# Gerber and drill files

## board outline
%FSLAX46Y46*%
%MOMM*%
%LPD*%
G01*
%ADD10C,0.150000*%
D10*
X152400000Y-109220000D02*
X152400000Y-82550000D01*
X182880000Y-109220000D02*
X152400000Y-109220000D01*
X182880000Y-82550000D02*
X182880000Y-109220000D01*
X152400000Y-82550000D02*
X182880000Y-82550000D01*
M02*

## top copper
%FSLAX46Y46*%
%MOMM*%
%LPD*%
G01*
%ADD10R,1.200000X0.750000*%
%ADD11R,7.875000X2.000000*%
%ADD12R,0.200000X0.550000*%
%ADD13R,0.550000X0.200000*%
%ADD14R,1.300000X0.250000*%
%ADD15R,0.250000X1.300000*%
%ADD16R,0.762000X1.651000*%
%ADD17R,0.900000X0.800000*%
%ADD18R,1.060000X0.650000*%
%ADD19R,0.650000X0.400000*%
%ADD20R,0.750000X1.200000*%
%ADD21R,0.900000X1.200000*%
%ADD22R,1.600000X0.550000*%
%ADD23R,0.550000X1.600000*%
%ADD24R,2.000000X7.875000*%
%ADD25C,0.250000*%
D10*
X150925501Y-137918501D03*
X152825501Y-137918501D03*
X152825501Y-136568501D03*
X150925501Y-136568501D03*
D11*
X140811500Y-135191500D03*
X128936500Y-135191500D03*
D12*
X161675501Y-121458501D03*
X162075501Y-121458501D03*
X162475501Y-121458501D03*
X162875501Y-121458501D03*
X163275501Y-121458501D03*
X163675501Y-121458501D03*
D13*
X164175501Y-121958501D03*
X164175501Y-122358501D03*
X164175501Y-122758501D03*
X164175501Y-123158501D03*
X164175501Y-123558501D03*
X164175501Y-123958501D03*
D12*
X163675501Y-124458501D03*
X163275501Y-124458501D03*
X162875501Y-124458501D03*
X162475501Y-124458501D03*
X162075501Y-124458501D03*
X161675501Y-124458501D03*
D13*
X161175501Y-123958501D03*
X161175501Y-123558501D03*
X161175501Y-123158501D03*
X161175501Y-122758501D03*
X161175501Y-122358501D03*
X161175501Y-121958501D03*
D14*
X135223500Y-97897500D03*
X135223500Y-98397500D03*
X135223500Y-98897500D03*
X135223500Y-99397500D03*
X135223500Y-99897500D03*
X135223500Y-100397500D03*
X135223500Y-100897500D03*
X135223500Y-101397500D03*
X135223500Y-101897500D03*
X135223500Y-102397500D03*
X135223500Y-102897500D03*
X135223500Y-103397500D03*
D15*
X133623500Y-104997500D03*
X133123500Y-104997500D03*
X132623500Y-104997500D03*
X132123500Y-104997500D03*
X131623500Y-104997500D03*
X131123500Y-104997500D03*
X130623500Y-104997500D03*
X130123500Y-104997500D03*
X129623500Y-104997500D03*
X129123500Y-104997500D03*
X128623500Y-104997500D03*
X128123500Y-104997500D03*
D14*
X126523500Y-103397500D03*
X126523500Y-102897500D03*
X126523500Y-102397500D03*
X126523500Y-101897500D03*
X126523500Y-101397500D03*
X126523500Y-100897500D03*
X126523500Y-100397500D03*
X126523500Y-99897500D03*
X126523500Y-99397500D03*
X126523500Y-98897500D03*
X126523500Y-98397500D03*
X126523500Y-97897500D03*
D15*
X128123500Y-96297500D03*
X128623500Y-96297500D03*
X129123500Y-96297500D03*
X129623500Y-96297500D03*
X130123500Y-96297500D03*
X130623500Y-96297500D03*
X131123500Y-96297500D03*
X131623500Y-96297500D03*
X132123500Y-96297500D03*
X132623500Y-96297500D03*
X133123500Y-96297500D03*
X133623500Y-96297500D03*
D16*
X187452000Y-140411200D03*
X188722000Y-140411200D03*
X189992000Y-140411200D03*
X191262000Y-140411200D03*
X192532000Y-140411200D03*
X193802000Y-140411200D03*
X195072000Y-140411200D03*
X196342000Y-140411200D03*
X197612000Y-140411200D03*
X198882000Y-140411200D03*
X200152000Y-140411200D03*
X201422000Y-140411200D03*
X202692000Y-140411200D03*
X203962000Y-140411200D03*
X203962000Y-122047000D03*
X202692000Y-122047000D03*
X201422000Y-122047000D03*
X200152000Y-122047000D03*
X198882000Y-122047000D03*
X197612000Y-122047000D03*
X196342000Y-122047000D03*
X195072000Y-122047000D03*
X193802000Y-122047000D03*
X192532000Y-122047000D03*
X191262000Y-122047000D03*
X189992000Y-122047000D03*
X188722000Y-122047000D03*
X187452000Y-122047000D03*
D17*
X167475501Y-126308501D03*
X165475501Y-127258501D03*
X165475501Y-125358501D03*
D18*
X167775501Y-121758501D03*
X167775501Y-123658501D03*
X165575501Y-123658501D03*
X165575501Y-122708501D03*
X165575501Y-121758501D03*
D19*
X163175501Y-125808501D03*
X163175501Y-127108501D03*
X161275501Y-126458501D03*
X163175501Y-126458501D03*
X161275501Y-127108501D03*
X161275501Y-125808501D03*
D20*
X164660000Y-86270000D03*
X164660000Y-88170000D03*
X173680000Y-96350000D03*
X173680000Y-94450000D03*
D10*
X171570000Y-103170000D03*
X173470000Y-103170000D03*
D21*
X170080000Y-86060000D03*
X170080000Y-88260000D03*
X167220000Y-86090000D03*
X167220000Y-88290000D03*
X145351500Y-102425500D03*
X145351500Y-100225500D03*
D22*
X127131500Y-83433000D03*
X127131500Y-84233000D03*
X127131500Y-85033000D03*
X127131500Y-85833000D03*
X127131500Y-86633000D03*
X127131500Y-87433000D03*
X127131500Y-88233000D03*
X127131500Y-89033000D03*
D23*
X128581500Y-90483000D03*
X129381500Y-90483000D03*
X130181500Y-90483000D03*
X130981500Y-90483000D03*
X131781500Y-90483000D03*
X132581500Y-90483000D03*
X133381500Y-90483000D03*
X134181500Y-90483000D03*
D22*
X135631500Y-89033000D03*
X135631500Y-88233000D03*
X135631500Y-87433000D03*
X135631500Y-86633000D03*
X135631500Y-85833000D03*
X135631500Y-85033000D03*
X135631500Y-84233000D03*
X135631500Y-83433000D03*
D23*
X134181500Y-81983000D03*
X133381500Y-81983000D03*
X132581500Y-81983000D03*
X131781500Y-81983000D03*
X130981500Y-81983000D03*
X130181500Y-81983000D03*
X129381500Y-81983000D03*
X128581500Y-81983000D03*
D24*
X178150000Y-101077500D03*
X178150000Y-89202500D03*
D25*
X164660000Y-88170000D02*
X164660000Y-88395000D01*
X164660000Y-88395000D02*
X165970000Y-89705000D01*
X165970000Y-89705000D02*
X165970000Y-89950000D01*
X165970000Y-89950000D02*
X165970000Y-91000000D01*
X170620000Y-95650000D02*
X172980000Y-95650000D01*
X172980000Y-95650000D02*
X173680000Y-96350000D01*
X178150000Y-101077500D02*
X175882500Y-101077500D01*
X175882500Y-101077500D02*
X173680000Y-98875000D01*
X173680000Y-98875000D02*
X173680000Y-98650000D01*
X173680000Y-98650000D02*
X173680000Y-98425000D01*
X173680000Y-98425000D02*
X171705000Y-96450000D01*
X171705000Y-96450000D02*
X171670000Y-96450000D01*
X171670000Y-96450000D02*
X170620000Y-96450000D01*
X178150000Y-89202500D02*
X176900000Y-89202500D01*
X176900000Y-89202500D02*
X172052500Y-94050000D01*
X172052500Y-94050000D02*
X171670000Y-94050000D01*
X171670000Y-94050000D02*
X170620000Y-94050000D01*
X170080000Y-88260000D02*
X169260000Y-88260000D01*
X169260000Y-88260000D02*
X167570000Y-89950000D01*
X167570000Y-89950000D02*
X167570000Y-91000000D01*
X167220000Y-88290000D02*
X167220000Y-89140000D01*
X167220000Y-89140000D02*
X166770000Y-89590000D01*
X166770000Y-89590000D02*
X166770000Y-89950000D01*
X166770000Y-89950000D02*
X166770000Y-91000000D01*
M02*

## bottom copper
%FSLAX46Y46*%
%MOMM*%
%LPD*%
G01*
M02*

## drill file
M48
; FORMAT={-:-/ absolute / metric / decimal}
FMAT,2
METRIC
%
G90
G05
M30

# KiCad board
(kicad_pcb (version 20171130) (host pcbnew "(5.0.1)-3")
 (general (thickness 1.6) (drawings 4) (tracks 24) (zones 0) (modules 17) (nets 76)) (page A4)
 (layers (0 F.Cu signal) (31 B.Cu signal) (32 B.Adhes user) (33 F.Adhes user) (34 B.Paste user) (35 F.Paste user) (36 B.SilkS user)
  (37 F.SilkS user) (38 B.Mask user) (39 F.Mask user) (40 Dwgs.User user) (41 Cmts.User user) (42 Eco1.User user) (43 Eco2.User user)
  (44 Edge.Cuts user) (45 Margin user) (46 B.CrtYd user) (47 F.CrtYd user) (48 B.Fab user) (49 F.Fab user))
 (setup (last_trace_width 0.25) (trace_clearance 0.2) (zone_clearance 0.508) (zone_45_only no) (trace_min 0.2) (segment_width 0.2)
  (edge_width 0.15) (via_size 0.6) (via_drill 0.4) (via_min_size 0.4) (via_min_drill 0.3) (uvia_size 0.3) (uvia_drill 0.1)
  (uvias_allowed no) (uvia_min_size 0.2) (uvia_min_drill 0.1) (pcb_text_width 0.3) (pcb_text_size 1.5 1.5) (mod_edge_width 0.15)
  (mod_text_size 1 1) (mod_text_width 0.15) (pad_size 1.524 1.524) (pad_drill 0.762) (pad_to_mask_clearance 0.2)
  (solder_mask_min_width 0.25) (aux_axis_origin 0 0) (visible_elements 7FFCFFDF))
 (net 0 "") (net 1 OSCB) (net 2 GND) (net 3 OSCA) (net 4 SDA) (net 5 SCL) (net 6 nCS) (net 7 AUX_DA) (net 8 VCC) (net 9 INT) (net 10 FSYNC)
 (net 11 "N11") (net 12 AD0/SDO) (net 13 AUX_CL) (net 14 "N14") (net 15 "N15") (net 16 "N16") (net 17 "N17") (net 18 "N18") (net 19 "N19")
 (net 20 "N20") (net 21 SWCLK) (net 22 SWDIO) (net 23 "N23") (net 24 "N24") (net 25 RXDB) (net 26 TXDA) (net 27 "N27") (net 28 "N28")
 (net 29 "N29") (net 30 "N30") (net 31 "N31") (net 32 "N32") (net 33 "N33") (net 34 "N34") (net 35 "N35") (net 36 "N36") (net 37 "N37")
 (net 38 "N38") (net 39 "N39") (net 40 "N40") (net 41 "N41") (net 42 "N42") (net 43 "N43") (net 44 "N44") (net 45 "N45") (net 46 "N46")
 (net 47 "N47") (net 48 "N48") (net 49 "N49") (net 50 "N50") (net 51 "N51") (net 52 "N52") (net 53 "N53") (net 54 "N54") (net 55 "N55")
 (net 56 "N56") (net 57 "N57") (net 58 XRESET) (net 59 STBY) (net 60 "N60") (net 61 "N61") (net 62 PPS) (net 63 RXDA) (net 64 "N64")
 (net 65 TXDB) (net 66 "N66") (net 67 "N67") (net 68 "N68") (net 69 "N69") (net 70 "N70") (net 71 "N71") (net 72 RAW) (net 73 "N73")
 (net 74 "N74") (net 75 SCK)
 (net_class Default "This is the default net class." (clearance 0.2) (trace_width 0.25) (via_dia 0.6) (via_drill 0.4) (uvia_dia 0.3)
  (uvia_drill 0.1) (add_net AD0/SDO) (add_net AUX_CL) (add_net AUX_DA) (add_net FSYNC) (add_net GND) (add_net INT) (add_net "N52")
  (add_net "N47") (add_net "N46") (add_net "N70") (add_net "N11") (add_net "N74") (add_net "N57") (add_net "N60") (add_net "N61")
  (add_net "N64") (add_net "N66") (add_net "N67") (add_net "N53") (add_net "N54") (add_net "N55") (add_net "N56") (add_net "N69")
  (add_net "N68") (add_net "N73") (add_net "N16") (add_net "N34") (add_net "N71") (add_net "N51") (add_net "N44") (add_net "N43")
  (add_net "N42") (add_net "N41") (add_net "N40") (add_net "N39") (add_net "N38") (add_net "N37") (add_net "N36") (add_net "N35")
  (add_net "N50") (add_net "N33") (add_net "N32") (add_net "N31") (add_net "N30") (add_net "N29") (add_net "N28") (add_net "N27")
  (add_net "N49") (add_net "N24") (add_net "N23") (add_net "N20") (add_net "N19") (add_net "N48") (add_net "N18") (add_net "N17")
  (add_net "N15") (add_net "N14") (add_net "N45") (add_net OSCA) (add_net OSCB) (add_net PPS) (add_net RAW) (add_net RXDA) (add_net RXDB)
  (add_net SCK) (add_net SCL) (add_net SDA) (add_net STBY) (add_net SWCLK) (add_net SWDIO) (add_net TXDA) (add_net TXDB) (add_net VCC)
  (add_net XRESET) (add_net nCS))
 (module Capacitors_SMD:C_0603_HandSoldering (layer F.Cu) (at 151.875501 137.918501)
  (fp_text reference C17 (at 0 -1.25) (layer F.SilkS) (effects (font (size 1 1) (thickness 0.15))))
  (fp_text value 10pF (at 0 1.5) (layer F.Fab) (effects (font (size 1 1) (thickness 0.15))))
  (pad 1 smd rect (at -0.95 0) (size 1.2 0.75) (layers F.Cu F.Paste F.Mask) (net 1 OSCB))
  (pad 2 smd rect (at 0.95 0) (size 1.2 0.75) (layers F.Cu F.Paste F.Mask) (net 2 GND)))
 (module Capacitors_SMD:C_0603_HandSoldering (layer F.Cu) (at 151.875501 136.568501)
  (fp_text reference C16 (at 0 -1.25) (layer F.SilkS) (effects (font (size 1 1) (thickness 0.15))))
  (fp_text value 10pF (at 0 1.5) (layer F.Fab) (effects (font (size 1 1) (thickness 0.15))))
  (pad 2 smd rect (at 0.95 0) (size 1.2 0.75) (layers F.Cu F.Paste F.Mask) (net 2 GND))
  (pad 1 smd rect (at -0.95 0) (size 1.2 0.75) (layers F.Cu F.Paste F.Mask) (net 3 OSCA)))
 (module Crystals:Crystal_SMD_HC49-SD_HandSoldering (layer F.Cu) (at 134.874 135.1915)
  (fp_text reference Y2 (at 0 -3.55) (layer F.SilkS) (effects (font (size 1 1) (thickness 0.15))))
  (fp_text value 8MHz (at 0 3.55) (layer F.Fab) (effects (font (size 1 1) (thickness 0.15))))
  (pad 2 smd rect (at 5.9375 0) (size 7.875 2) (layers F.Cu F.Paste F.Mask) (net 1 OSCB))
  (pad 1 smd rect (at -5.9375 0) (size 7.875 2) (layers F.Cu F.Paste F.Mask) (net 3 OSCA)))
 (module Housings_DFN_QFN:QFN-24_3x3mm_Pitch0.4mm (layer F.Cu) (at 162.675501 122.958501)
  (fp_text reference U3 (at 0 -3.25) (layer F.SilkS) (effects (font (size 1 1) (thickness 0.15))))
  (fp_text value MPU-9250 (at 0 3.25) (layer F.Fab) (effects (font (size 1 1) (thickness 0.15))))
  (pad 24 smd rect (at -1 -1.5 90) (size 0.55 0.2) (layers F.Cu F.Paste F.Mask) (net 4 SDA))
  (pad 23 smd rect (at -0.6 -1.5 90) (size 0.55 0.2) (layers F.Cu F.Paste F.Mask) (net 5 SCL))
  (pad 22 smd rect (at -0.2 -1.5 90) (size 0.55 0.2) (layers F.Cu F.Paste F.Mask) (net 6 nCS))
  (pad 21 smd rect (at 0.2 -1.5 90) (size 0.55 0.2) (layers F.Cu F.Paste F.Mask) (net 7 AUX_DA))
  (pad 20 smd rect (at 0.6 -1.5 90) (size 0.55 0.2) (layers F.Cu F.Paste F.Mask))
  (pad 19 smd rect (at 1 -1.5 90) (size 0.55 0.2) (layers F.Cu F.Paste F.Mask))
  (pad 18 smd rect (at 1.5 -1) (size 0.55 0.2) (layers F.Cu F.Paste F.Mask) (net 2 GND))
  (pad 17 smd rect (at 1.5 -0.6) (size 0.55 0.2) (layers F.Cu F.Paste F.Mask))
  (pad 16 smd rect (at 1.5 -0.2) (size 0.55 0.2) (layers F.Cu F.Paste F.Mask))
  (pad 15 smd rect (at 1.5 0.2) (size 0.55 0.2) (layers F.Cu F.Paste F.Mask))
  (pad 14 smd rect (at 1.5 0.6) (size 0.55 0.2) (layers F.Cu F.Paste F.Mask))
  (pad 13 smd rect (at 1.5 1) (size 0.55 0.2) (layers F.Cu F.Paste F.Mask) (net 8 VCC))
  (pad 12 smd rect (at 1 1.5 90) (size 0.55 0.2) (layers F.Cu F.Paste F.Mask) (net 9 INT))
  (pad 11 smd rect (at 0.6 1.5 90) (size 0.55 0.2) (layers F.Cu F.Paste F.Mask) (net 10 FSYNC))
  (pad 10 smd rect (at 0.2 1.5 90) (size 0.55 0.2) (layers F.Cu F.Paste F.Mask) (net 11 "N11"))
  (pad 9 smd rect (at -0.2 1.5 90) (size 0.55 0.2) (layers F.Cu F.Paste F.Mask) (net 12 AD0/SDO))
  (pad 8 smd rect (at -0.6 1.5 90) (size 0.55 0.2) (layers F.Cu F.Paste F.Mask) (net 8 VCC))
  (pad 7 smd rect (at -1 1.5 90) (size 0.55 0.2) (layers F.Cu F.Paste F.Mask) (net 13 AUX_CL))
  (pad 6 smd rect (at -1.5 1) (size 0.55 0.2) (layers F.Cu F.Paste F.Mask))
  (pad 5 smd rect (at -1.5 0.6) (size 0.55 0.2) (layers F.Cu F.Paste F.Mask))
  (pad 4 smd rect (at -1.5 0.2) (size 0.55 0.2) (layers F.Cu F.Paste F.Mask))
  (pad 3 smd rect (at -1.5 -0.2) (size 0.55 0.2) (layers F.Cu F.Paste F.Mask))
  (pad 2 smd rect (at -1.5 -0.6) (size 0.55 0.2) (layers F.Cu F.Paste F.Mask))
  (pad 1 smd rect (at -1.5 -1) (size 0.55 0.2) (layers F.Cu F.Paste F.Mask)))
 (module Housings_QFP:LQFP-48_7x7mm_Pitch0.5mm (layer F.Cu) (at 130.8735 100.6475 270)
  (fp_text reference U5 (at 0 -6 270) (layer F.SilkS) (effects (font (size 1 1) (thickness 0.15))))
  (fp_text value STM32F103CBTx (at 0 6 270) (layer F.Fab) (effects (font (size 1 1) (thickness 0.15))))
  (pad 48 smd rect (at -2.75 -4.35) (size 1.3 0.25) (layers F.Cu F.Paste F.Mask) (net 8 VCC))
  (pad 47 smd rect (at -2.25 -4.35) (size 1.3 0.25) (layers F.Cu F.Paste F.Mask) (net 2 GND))
  (pad 46 smd rect (at -1.75 -4.35) (size 1.3 0.25) (layers F.Cu F.Paste F.Mask) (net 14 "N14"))
  (pad 45 smd rect (at -1.25 -4.35) (size 1.3 0.25) (layers F.Cu F.Paste F.Mask) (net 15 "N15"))
  (pad 44 smd rect (at -0.75 -4.35) (size 1.3 0.25) (layers F.Cu F.Paste F.Mask) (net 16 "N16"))
  (pad 43 smd rect (at -0.25 -4.35) (size 1.3 0.25) (layers F.Cu F.Paste F.Mask) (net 4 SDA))
  (pad 42 smd rect (at 0.25 -4.35) (size 1.3 0.25) (layers F.Cu F.Paste F.Mask) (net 5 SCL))
  (pad 41 smd rect (at 0.75 -4.35) (size 1.3 0.25) (layers F.Cu F.Paste F.Mask) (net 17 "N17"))
  (pad 40 smd rect (at 1.25 -4.35) (size 1.3 0.25) (layers F.Cu F.Paste F.Mask) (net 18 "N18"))
  (pad 39 smd rect (at 1.75 -4.35) (size 1.3 0.25) (layers F.Cu F.Paste F.Mask) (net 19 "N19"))
  (pad 38 smd rect (at 2.25 -4.35) (size 1.3 0.25) (layers F.Cu F.Paste F.Mask) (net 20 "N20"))
  (pad 37 smd rect (at 2.75 -4.35) (size 1.3 0.25) (layers F.Cu F.Paste F.Mask) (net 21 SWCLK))
  (pad 36 smd rect (at 4.35 -2.75 270) (size 1.3 0.25) (layers F.Cu F.Paste F.Mask) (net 8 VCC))
  (pad 35 smd rect (at 4.35 -2.25 270) (size 1.3 0.25) (layers F.Cu F.Paste F.Mask) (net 2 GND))
  (pad 34 smd rect (at 4.35 -1.75 270) (size 1.3 0.25) (layers F.Cu F.Paste F.Mask) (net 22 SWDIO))
  (pad 33 smd rect (at 4.35 -1.25 270) (size 1.3 0.25) (layers F.Cu F.Paste F.Mask) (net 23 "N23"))
  (pad 32 smd rect (at 4.35 -0.75 270) (size 1.3 0.25) (layers F.Cu F.Paste F.Mask) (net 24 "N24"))
  (pad 31 smd rect (at 4.35 -0.25 270) (size 1.3 0.25) (layers F.Cu F.Paste F.Mask) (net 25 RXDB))
  (pad 30 smd rect (at 4.35 0.25 270) (size 1.3 0.25) (layers F.Cu F.Paste F.Mask) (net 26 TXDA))
  (pad 29 smd rect (at 4.35 0.75 270) (size 1.3 0.25) (layers F.Cu F.Paste F.Mask) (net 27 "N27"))
  (pad 28 smd rect (at 4.35 1.25 270) (size 1.3 0.25) (layers F.Cu F.Paste F.Mask) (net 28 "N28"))
  (pad 27 smd rect (at 4.35 1.75 270) (size 1.3 0.25) (layers F.Cu F.Paste F.Mask) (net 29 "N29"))
  (pad 26 smd rect (at 4.35 2.25 270) (size 1.3 0.25) (layers F.Cu F.Paste F.Mask) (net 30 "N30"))
  (pad 25 smd rect (at 4.35 2.75 270) (size 1.3 0.25) (layers F.Cu F.Paste F.Mask) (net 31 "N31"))
  (pad 24 smd rect (at 2.75 4.35) (size 1.3 0.25) (layers F.Cu F.Paste F.Mask) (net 8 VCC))
  (pad 23 smd rect (at 2.25 4.35) (size 1.3 0.25) (layers F.Cu F.Paste F.Mask) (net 2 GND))
  (pad 22 smd rect (at 1.75 4.35) (size 1.3 0.25) (layers F.Cu F.Paste F.Mask) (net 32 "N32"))
  (pad 21 smd rect (at 1.25 4.35) (size 1.3 0.25) (layers F.Cu F.Paste F.Mask) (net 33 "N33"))
  (pad 20 smd rect (at 0.75 4.35) (size 1.3 0.25) (layers F.Cu F.Paste F.Mask) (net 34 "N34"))
  (pad 19 smd rect (at 0.25 4.35) (size 1.3 0.25) (layers F.Cu F.Paste F.Mask) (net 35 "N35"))
  (pad 18 smd rect (at -0.25 4.35) (size 1.3 0.25) (layers F.Cu F.Paste F.Mask) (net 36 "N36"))
  (pad 17 smd rect (at -0.75 4.35) (size 1.3 0.25) (layers F.Cu F.Paste F.Mask) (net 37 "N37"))
  (pad 16 smd rect (at -1.25 4.35) (size 1.3 0.25) (layers F.Cu F.Paste F.Mask) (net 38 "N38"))
  (pad 15 smd rect (at -1.75 4.35) (size 1.3 0.25) (layers F.Cu F.Paste F.Mask) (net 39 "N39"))
  (pad 14 smd rect (at -2.25 4.35) (size 1.3 0.25) (layers F.Cu F.Paste F.Mask) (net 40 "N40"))
  (pad 13 smd rect (at -2.75 4.35) (size 1.3 0.25) (layers F.Cu F.Paste F.Mask) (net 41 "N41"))
  (pad 12 smd rect (at -4.35 2.75 270) (size 1.3 0.25) (layers F.Cu F.Paste F.Mask) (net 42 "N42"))
  (pad 11 smd rect (at -4.35 2.25 270) (size 1.3 0.25) (layers F.Cu F.Paste F.Mask) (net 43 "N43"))
  (pad 10 smd rect (at -4.35 1.75 270) (size 1.3 0.25) (layers F.Cu F.Paste F.Mask) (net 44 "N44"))
  (pad 9 smd rect (at -4.35 1.25 270) (size 1.3 0.25) (layers F.Cu F.Paste F.Mask) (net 8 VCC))
  (pad 8 smd rect (at -4.35 0.75 270) (size 1.3 0.25) (layers F.Cu F.Paste F.Mask) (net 2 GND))
  (pad 7 smd rect (at -4.35 0.25 270) (size 1.3 0.25) (layers F.Cu F.Paste F.Mask) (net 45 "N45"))
  (pad 6 smd rect (at -4.35 -0.25 270) (size 1.3 0.25) (layers F.Cu F.Paste F.Mask) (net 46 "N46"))
  (pad 5 smd rect (at -4.35 -0.75 270) (size 1.3 0.25) (layers F.Cu F.Paste F.Mask) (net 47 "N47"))
  (pad 4 smd rect (at -4.35 -1.25 270) (size 1.3 0.25) (layers F.Cu F.Paste F.Mask) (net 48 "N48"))
  (pad 3 smd rect (at -4.35 -1.75 270) (size 1.3 0.25) (layers F.Cu F.Paste F.Mask) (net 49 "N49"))
  (pad 2 smd rect (at -4.35 -2.25 270) (size 1.3 0.25) (layers F.Cu F.Paste F.Mask) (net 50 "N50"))
  (pad 1 smd rect (at -4.35 -2.75 270) (size 1.3 0.25) (layers F.Cu F.Paste F.Mask) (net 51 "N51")))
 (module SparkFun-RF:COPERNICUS (layer F.Cu) (at 187.452 122.047)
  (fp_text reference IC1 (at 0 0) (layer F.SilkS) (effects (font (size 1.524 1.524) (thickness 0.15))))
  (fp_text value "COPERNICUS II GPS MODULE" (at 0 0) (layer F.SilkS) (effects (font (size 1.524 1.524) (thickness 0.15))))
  (pad 1 smd rect (at 0 18.3642 180) (size 0.762 1.651) (layers F.Cu F.Paste F.Mask) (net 2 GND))
  (pad 2 smd rect (at 1.27 18.3642 180) (size 0.762 1.651) (layers F.Cu F.Paste F.Mask) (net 2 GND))
  (pad 3 smd rect (at 2.54 18.3642 180) (size 0.762 1.651) (layers F.Cu F.Paste F.Mask) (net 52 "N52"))
  (pad 4 smd rect (at 3.81 18.3642 180) (size 0.762 1.651) (layers F.Cu F.Paste F.Mask) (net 2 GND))
  (pad 5 smd rect (at 5.08 18.3642 180) (size 0.762 1.651) (layers F.Cu F.Paste F.Mask) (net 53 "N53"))
  (pad 6 smd rect (at 6.35 18.3642 180) (size 0.762 1.651) (layers F.Cu F.Paste F.Mask) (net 8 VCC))
  (pad 7 smd rect (at 7.62 18.3642 180) (size 0.762 1.651) (layers F.Cu F.Paste F.Mask) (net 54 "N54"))
  (pad 8 smd rect (at 8.89 18.3642 180) (size 0.762 1.651) (layers F.Cu F.Paste F.Mask) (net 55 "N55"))
  (pad 9 smd rect (at 10.16 18.3642 180) (size 0.762 1.651) (layers F.Cu F.Paste F.Mask) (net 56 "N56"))
  (pad 10 smd rect (at 11.43 18.3642 180) (size 0.762 1.651) (layers F.Cu F.Paste F.Mask) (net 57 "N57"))
  (pad 11 smd rect (at 12.7 18.3642 180) (size 0.762 1.651) (layers F.Cu F.Paste F.Mask) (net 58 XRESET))
  (pad 12 smd rect (at 13.97 18.3642 180) (size 0.762 1.651) (layers F.Cu F.Paste F.Mask) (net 8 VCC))
  (pad 13 smd rect (at 15.24 18.3642 180) (size 0.762 1.651) (layers F.Cu F.Paste F.Mask) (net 2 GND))
  (pad 14 smd rect (at 16.51 18.3642 180) (size 0.762 1.651) (layers F.Cu F.Paste F.Mask) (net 2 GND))
  (pad 15 smd rect (at 16.51 0 180) (size 0.762 1.651) (layers F.Cu F.Paste F.Mask) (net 2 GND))
  (pad 16 smd rect (at 15.24 0 180) (size 0.762 1.651) (layers F.Cu F.Paste F.Mask) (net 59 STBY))
  (pad 17 smd rect (at 13.97 0 180) (size 0.762 1.651) (layers F.Cu F.Paste F.Mask) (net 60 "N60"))
  (pad 18 smd rect (at 12.7 0 180) (size 0.762 1.651) (layers F.Cu F.Paste F.Mask) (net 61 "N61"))
  (pad 19 smd rect (at 11.43 0 180) (size 0.762 1.651) (layers F.Cu F.Paste F.Mask) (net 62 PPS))
  (pad 20 smd rect (at 10.16 0 180) (size 0.762 1.651) (layers F.Cu F.Paste F.Mask) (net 25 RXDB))
  (pad 21 smd rect (at 8.89 0 180) (size 0.762 1.651) (layers F.Cu F.Paste F.Mask) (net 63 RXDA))
  (pad 22 smd rect (at 7.62 0 180) (size 0.762 1.651) (layers F.Cu F.Paste F.Mask) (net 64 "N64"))
  (pad 23 smd rect (at 6.35 0 180) (size 0.762 1.651) (layers F.Cu F.Paste F.Mask) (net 26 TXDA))
  (pad 24 smd rect (at 5.08 0 180) (size 0.762 1.651) (layers F.Cu F.Paste F.Mask) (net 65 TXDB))
  (pad 25 smd rect (at 3.81 0 180) (size 0.762 1.651) (layers F.Cu F.Paste F.Mask) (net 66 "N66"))
  (pad 26 smd rect (at 2.54 0 180) (size 0.762 1.651) (layers F.Cu F.Paste F.Mask) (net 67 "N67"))
  (pad 27 smd rect (at 1.27 0 180) (size 0.762 1.651) (layers F.Cu F.Paste F.Mask) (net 2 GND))
  (pad 28 smd rect (at 0 0 180) (size 0.762 1.651) (layers F.Cu F.Paste F.Mask) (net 2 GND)))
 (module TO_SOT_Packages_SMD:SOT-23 (layer F.Cu) (at 166.475501 126.308501)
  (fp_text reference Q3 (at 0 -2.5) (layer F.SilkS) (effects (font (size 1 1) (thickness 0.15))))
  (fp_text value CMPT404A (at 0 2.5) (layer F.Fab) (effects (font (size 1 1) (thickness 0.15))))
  (pad 3 smd rect (at 1 0) (size 0.9 0.8) (layers F.Cu F.Paste F.Mask) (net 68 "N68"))
  (pad 2 smd rect (at -1 0.95) (size 0.9 0.8) (layers F.Cu F.Paste F.Mask) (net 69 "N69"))
  (pad 1 smd rect (at -1 -0.95) (size 0.9 0.8) (layers F.Cu F.Paste F.Mask) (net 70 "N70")))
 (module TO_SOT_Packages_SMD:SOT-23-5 (layer F.Cu) (at 166.675501 122.708501)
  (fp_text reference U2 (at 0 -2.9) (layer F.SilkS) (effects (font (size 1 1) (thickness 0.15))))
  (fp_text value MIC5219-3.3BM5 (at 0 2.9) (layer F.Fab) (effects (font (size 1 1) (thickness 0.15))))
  (pad 5 smd rect (at 1.1 -0.95) (size 1.06 0.65) (layers F.Cu F.Paste F.Mask) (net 8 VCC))
  (pad 4 smd rect (at 1.1 0.95) (size 1.06 0.65) (layers F.Cu F.Paste F.Mask) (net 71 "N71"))
  (pad 3 smd rect (at -1.1 0.95) (size 1.06 0.65) (layers F.Cu F.Paste F.Mask) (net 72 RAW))
  (pad 2 smd rect (at -1.1 0) (size 1.06 0.65) (layers F.Cu F.Paste F.Mask) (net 2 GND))
  (pad 1 smd rect (at -1.1 -0.95) (size 1.06 0.65) (layers F.Cu F.Paste F.Mask) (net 72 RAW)))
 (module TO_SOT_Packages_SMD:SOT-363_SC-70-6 (layer F.Cu) (at 162.225501 126.458501)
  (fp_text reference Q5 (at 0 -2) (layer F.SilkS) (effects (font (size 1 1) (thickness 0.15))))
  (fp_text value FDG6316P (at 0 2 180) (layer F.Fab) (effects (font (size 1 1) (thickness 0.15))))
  (pad 6 smd rect (at 0.95 -0.65) (size 0.65 0.4) (layers F.Cu F.Paste F.Mask))
  (pad 4 smd rect (at 0.95 0.65) (size 0.65 0.4) (layers F.Cu F.Paste F.Mask))
  (pad 2 smd rect (at -0.95 0) (size 0.65 0.4) (layers F.Cu F.Paste F.Mask) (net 53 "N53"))
  (pad 5 smd rect (at 0.95 0) (size 0.65 0.4) (layers F.Cu F.Paste F.Mask))
  (pad 3 smd rect (at -0.95 0.65) (size 0.65 0.4) (layers F.Cu F.Paste F.Mask) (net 8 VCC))
  (pad 1 smd rect (at -0.95 -0.65) (size 0.65 0.4) (layers F.Cu F.Paste F.Mask) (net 69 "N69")))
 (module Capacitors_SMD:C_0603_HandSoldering (layer F.Cu) (at 164.66 87.22 270)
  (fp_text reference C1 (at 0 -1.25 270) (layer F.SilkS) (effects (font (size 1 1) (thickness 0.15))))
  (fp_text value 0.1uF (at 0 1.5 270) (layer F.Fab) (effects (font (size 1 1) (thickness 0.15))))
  (pad 1 smd rect (at -0.95 0 270) (size 1.2 0.75) (layers F.Cu F.Paste F.Mask) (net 8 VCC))
  (pad 2 smd rect (at 0.95 0 270) (size 1.2 0.75) (layers F.Cu F.Paste F.Mask) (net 2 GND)))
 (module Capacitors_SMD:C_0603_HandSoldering (layer F.Cu) (at 173.68 95.4 90)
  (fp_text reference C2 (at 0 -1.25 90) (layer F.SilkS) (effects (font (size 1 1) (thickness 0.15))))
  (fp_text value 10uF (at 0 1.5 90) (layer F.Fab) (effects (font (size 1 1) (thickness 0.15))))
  (pad 1 smd rect (at -0.95 0 90) (size 1.2 0.75) (layers F.Cu F.Paste F.Mask) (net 72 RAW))
  (pad 2 smd rect (at 0.95 0 90) (size 1.2 0.75) (layers F.Cu F.Paste F.Mask) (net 2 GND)))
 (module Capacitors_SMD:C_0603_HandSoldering (layer F.Cu) (at 172.52 103.17)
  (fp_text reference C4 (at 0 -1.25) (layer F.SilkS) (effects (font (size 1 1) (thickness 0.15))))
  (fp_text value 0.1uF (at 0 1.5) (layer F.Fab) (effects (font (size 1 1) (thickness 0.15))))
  (pad 1 smd rect (at -0.95 0) (size 1.2 0.75) (layers F.Cu F.Paste F.Mask) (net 11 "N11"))
  (pad 2 smd rect (at 0.95 0) (size 1.2 0.75) (layers F.Cu F.Paste F.Mask) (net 2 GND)))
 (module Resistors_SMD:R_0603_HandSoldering (layer F.Cu) (at 170.08 87.16 270)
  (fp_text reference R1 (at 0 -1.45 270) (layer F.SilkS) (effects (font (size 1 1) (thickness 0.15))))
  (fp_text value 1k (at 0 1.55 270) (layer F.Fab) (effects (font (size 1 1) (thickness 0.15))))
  (pad 1 smd rect (at -1.1 0 270) (size 1.2 0.9) (layers F.Cu F.Paste F.Mask) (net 70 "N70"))
  (pad 2 smd rect (at 1.1 0 270) (size 1.2 0.9) (layers F.Cu F.Paste F.Mask) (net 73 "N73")))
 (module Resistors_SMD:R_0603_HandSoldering (layer F.Cu) (at 167.22 87.19 270)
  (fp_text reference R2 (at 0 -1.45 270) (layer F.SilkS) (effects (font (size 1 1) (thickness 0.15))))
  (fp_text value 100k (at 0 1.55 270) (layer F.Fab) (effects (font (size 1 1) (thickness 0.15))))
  (pad 1 smd rect (at -1.1 0 270) (size 1.2 0.9) (layers F.Cu F.Paste F.Mask) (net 8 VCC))
  (pad 2 smd rect (at 1.1 0 270) (size 1.2 0.9) (layers F.Cu F.Paste F.Mask) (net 53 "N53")))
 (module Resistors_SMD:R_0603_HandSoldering (layer F.Cu) (at 145.3515 101.3255 90)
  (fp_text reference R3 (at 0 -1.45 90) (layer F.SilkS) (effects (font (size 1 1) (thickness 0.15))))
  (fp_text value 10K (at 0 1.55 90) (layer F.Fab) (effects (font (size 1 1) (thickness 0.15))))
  (pad 1 smd rect (at -1.1 0 90) (size 1.2 0.9) (layers F.Cu F.Paste F.Mask) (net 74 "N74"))
  (pad 2 smd rect (at 1.1 0 90) (size 1.2 0.9) (layers F.Cu F.Paste F.Mask) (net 2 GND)))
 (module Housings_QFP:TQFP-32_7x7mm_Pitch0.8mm (layer F.Cu) (at 131.3815 86.233)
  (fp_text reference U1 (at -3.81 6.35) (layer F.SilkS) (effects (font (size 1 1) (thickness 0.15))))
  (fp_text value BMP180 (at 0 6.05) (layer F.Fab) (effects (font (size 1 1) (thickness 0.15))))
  (pad 1 smd rect (at -4.25 -2.8) (size 1.6 0.55) (layers F.Cu F.Paste F.Mask))
  (pad 2 smd rect (at -4.25 -2) (size 1.6 0.55) (layers F.Cu F.Paste F.Mask) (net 8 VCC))
  (pad 3 smd rect (at -4.25 -1.2) (size 1.6 0.55) (layers F.Cu F.Paste F.Mask) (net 8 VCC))
  (pad 4 smd rect (at -4.25 -0.4) (size 1.6 0.55) (layers F.Cu F.Paste F.Mask))
  (pad 5 smd rect (at -4.25 0.4) (size 1.6 0.55) (layers F.Cu F.Paste F.Mask) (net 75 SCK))
  (pad 6 smd rect (at -4.25 1.2) (size 1.6 0.55) (layers F.Cu F.Paste F.Mask) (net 4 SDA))
  (pad 7 smd rect (at -4.25 2) (size 1.6 0.55) (layers F.Cu F.Paste F.Mask) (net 2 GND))
  (pad 8 smd rect (at -4.25 2.8) (size 1.6 0.55) (layers F.Cu F.Paste F.Mask))
  (pad 9 smd rect (at -2.8 4.25 90) (size 1.6 0.55) (layers F.Cu F.Paste F.Mask))
  (pad 10 smd rect (at -2 4.25 90) (size 1.6 0.55) (layers F.Cu F.Paste F.Mask))
  (pad 11 smd rect (at -1.2 4.25 90) (size 1.6 0.55) (layers F.Cu F.Paste F.Mask))
  (pad 12 smd rect (at -0.4 4.25 90) (size 1.6 0.55) (layers F.Cu F.Paste F.Mask))
  (pad 13 smd rect (at 0.4 4.25 90) (size 1.6 0.55) (layers F.Cu F.Paste F.Mask))
  (pad 14 smd rect (at 1.2 4.25 90) (size 1.6 0.55) (layers F.Cu F.Paste F.Mask))
  (pad 15 smd rect (at 2 4.25 90) (size 1.6 0.55) (layers F.Cu F.Paste F.Mask))
  (pad 16 smd rect (at 2.8 4.25 90) (size 1.6 0.55) (layers F.Cu F.Paste F.Mask))
  (pad 17 smd rect (at 4.25 2.8) (size 1.6 0.55) (layers F.Cu F.Paste F.Mask))
  (pad 18 smd rect (at 4.25 2) (size 1.6 0.55) (layers F.Cu F.Paste F.Mask))
  (pad 19 smd rect (at 4.25 1.2) (size 1.6 0.55) (layers F.Cu F.Paste F.Mask))
  (pad 20 smd rect (at 4.25 0.4) (size 1.6 0.55) (layers F.Cu F.Paste F.Mask))
  (pad 21 smd rect (at 4.25 -0.4) (size 1.6 0.55) (layers F.Cu F.Paste F.Mask))
  (pad 22 smd rect (at 4.25 -1.2) (size 1.6 0.55) (layers F.Cu F.Paste F.Mask))
  (pad 23 smd rect (at 4.25 -2) (size 1.6 0.55) (layers F.Cu F.Paste F.Mask))
  (pad 24 smd rect (at 4.25 -2.8) (size 1.6 0.55) (layers F.Cu F.Paste F.Mask))
  (pad 25 smd rect (at 2.8 -4.25 90) (size 1.6 0.55) (layers F.Cu F.Paste F.Mask))
  (pad 26 smd rect (at 2 -4.25 90) (size 1.6 0.55) (layers F.Cu F.Paste F.Mask))
  (pad 27 smd rect (at 1.2 -4.25 90) (size 1.6 0.55) (layers F.Cu F.Paste F.Mask))
  (pad 28 smd rect (at 0.4 -4.25 90) (size 1.6 0.55) (layers F.Cu F.Paste F.Mask))
  (pad 29 smd rect (at -0.4 -4.25 90) (size 1.6 0.55) (layers F.Cu F.Paste F.Mask))
  (pad 30 smd rect (at -1.2 -4.25 90) (size 1.6 0.55) (layers F.Cu F.Paste F.Mask))
  (pad 31 smd rect (at -2 -4.25 90) (size 1.6 0.55) (layers F.Cu F.Paste F.Mask))
  (pad 32 smd rect (at -2.8 -4.25 90) (size 1.6 0.55) (layers F.Cu F.Paste F.Mask)))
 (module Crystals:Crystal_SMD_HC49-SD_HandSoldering (layer F.Cu) (at 178.15 95.14 90)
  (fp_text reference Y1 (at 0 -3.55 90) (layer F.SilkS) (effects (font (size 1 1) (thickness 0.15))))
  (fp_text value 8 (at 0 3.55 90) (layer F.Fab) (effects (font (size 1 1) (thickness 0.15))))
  (pad 1 smd rect (at -5.9375 0 90) (size 7.875 2) (layers F.Cu F.Paste F.Mask) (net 47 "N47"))
  (pad 2 smd rect (at 5.9375 0 90) (size 7.875 2) (layers F.Cu F.Paste F.Mask) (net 46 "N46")))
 (gr_line (start 152.4 109.22) (end 152.4 82.55) (layer Edge.Cuts) (width 0.15))
 (gr_line (start 182.88 109.22) (end 152.4 109.22) (layer Edge.Cuts) (width 0.15))
 (gr_line (start 182.88 82.55) (end 182.88 109.22) (layer Edge.Cuts) (width 0.15))
 (gr_line (start 152.4 82.55) (end 182.88 82.55) (layer Edge.Cuts) (width 0.15))
 (segment (start 164.66 88.17) (end 164.66 88.395) (width 0.25) (layer F.Cu) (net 2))
 (segment (start 164.66 88.395) (end 165.97 89.705) (width 0.25) (layer F.Cu) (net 2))
 (segment (start 165.97 89.705) (end 165.97 89.95) (width 0.25) (layer F.Cu) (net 2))
 (segment (start 165.97 89.95) (end 165.97 91) (width 0.25) (layer F.Cu) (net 2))
 (segment (start 170.62 95.65) (end 172.98 95.65) (width 0.25) (layer F.Cu) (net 72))
 (segment (start 172.98 95.65) (end 173.68 96.35) (width 0.25) (layer F.Cu) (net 72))
 (segment (start 178.15 101.0775) (end 175.8825 101.0775) (width 0.25) (layer F.Cu) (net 47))
 (segment (start 175.8825 101.0775) (end 173.68 98.875) (width 0.25) (layer F.Cu) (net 47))
 (segment (start 173.68 98.875) (end 173.68 98.65) (width 0.25) (layer F.Cu) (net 47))
 (segment (start 173.68 98.65) (end 173.68 98.425) (width 0.25) (layer F.Cu) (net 47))
 (segment (start 173.68 98.425) (end 171.705 96.45) (width 0.25) (layer F.Cu) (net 47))
 (segment (start 171.705 96.45) (end 171.67 96.45) (width 0.25) (layer F.Cu) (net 47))
 (segment (start 171.67 96.45) (end 170.62 96.45) (width 0.25) (layer F.Cu) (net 47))
 (segment (start 178.15 89.2025) (end 176.9 89.2025) (width 0.25) (layer F.Cu) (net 46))
 (segment (start 176.9 89.2025) (end 172.0525 94.05) (width 0.25) (layer F.Cu) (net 46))
 (segment (start 172.0525 94.05) (end 171.67 94.05) (width 0.25) (layer F.Cu) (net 46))
 (segment (start 171.67 94.05) (end 170.62 94.05) (width 0.25) (layer F.Cu) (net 46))
 (segment (start 170.08 88.26) (end 169.26 88.26) (width 0.25) (layer F.Cu) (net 73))
 (segment (start 169.26 88.26) (end 167.57 89.95) (width 0.25) (layer F.Cu) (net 73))
 (segment (start 167.57 89.95) (end 167.57 91) (width 0.25) (layer F.Cu) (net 73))
 (segment (start 167.22 88.29) (end 167.22 89.14) (width 0.25) (layer F.Cu) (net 53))
 (segment (start 167.22 89.14) (end 166.77 89.59) (width 0.25) (layer F.Cu) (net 53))
 (segment (start 166.77 89.59) (end 166.77 89.95) (width 0.25) (layer F.Cu) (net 53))
 (segment (start 166.77 89.95) (end 166.77 91) (width 0.25) (layer F.Cu) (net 53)))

